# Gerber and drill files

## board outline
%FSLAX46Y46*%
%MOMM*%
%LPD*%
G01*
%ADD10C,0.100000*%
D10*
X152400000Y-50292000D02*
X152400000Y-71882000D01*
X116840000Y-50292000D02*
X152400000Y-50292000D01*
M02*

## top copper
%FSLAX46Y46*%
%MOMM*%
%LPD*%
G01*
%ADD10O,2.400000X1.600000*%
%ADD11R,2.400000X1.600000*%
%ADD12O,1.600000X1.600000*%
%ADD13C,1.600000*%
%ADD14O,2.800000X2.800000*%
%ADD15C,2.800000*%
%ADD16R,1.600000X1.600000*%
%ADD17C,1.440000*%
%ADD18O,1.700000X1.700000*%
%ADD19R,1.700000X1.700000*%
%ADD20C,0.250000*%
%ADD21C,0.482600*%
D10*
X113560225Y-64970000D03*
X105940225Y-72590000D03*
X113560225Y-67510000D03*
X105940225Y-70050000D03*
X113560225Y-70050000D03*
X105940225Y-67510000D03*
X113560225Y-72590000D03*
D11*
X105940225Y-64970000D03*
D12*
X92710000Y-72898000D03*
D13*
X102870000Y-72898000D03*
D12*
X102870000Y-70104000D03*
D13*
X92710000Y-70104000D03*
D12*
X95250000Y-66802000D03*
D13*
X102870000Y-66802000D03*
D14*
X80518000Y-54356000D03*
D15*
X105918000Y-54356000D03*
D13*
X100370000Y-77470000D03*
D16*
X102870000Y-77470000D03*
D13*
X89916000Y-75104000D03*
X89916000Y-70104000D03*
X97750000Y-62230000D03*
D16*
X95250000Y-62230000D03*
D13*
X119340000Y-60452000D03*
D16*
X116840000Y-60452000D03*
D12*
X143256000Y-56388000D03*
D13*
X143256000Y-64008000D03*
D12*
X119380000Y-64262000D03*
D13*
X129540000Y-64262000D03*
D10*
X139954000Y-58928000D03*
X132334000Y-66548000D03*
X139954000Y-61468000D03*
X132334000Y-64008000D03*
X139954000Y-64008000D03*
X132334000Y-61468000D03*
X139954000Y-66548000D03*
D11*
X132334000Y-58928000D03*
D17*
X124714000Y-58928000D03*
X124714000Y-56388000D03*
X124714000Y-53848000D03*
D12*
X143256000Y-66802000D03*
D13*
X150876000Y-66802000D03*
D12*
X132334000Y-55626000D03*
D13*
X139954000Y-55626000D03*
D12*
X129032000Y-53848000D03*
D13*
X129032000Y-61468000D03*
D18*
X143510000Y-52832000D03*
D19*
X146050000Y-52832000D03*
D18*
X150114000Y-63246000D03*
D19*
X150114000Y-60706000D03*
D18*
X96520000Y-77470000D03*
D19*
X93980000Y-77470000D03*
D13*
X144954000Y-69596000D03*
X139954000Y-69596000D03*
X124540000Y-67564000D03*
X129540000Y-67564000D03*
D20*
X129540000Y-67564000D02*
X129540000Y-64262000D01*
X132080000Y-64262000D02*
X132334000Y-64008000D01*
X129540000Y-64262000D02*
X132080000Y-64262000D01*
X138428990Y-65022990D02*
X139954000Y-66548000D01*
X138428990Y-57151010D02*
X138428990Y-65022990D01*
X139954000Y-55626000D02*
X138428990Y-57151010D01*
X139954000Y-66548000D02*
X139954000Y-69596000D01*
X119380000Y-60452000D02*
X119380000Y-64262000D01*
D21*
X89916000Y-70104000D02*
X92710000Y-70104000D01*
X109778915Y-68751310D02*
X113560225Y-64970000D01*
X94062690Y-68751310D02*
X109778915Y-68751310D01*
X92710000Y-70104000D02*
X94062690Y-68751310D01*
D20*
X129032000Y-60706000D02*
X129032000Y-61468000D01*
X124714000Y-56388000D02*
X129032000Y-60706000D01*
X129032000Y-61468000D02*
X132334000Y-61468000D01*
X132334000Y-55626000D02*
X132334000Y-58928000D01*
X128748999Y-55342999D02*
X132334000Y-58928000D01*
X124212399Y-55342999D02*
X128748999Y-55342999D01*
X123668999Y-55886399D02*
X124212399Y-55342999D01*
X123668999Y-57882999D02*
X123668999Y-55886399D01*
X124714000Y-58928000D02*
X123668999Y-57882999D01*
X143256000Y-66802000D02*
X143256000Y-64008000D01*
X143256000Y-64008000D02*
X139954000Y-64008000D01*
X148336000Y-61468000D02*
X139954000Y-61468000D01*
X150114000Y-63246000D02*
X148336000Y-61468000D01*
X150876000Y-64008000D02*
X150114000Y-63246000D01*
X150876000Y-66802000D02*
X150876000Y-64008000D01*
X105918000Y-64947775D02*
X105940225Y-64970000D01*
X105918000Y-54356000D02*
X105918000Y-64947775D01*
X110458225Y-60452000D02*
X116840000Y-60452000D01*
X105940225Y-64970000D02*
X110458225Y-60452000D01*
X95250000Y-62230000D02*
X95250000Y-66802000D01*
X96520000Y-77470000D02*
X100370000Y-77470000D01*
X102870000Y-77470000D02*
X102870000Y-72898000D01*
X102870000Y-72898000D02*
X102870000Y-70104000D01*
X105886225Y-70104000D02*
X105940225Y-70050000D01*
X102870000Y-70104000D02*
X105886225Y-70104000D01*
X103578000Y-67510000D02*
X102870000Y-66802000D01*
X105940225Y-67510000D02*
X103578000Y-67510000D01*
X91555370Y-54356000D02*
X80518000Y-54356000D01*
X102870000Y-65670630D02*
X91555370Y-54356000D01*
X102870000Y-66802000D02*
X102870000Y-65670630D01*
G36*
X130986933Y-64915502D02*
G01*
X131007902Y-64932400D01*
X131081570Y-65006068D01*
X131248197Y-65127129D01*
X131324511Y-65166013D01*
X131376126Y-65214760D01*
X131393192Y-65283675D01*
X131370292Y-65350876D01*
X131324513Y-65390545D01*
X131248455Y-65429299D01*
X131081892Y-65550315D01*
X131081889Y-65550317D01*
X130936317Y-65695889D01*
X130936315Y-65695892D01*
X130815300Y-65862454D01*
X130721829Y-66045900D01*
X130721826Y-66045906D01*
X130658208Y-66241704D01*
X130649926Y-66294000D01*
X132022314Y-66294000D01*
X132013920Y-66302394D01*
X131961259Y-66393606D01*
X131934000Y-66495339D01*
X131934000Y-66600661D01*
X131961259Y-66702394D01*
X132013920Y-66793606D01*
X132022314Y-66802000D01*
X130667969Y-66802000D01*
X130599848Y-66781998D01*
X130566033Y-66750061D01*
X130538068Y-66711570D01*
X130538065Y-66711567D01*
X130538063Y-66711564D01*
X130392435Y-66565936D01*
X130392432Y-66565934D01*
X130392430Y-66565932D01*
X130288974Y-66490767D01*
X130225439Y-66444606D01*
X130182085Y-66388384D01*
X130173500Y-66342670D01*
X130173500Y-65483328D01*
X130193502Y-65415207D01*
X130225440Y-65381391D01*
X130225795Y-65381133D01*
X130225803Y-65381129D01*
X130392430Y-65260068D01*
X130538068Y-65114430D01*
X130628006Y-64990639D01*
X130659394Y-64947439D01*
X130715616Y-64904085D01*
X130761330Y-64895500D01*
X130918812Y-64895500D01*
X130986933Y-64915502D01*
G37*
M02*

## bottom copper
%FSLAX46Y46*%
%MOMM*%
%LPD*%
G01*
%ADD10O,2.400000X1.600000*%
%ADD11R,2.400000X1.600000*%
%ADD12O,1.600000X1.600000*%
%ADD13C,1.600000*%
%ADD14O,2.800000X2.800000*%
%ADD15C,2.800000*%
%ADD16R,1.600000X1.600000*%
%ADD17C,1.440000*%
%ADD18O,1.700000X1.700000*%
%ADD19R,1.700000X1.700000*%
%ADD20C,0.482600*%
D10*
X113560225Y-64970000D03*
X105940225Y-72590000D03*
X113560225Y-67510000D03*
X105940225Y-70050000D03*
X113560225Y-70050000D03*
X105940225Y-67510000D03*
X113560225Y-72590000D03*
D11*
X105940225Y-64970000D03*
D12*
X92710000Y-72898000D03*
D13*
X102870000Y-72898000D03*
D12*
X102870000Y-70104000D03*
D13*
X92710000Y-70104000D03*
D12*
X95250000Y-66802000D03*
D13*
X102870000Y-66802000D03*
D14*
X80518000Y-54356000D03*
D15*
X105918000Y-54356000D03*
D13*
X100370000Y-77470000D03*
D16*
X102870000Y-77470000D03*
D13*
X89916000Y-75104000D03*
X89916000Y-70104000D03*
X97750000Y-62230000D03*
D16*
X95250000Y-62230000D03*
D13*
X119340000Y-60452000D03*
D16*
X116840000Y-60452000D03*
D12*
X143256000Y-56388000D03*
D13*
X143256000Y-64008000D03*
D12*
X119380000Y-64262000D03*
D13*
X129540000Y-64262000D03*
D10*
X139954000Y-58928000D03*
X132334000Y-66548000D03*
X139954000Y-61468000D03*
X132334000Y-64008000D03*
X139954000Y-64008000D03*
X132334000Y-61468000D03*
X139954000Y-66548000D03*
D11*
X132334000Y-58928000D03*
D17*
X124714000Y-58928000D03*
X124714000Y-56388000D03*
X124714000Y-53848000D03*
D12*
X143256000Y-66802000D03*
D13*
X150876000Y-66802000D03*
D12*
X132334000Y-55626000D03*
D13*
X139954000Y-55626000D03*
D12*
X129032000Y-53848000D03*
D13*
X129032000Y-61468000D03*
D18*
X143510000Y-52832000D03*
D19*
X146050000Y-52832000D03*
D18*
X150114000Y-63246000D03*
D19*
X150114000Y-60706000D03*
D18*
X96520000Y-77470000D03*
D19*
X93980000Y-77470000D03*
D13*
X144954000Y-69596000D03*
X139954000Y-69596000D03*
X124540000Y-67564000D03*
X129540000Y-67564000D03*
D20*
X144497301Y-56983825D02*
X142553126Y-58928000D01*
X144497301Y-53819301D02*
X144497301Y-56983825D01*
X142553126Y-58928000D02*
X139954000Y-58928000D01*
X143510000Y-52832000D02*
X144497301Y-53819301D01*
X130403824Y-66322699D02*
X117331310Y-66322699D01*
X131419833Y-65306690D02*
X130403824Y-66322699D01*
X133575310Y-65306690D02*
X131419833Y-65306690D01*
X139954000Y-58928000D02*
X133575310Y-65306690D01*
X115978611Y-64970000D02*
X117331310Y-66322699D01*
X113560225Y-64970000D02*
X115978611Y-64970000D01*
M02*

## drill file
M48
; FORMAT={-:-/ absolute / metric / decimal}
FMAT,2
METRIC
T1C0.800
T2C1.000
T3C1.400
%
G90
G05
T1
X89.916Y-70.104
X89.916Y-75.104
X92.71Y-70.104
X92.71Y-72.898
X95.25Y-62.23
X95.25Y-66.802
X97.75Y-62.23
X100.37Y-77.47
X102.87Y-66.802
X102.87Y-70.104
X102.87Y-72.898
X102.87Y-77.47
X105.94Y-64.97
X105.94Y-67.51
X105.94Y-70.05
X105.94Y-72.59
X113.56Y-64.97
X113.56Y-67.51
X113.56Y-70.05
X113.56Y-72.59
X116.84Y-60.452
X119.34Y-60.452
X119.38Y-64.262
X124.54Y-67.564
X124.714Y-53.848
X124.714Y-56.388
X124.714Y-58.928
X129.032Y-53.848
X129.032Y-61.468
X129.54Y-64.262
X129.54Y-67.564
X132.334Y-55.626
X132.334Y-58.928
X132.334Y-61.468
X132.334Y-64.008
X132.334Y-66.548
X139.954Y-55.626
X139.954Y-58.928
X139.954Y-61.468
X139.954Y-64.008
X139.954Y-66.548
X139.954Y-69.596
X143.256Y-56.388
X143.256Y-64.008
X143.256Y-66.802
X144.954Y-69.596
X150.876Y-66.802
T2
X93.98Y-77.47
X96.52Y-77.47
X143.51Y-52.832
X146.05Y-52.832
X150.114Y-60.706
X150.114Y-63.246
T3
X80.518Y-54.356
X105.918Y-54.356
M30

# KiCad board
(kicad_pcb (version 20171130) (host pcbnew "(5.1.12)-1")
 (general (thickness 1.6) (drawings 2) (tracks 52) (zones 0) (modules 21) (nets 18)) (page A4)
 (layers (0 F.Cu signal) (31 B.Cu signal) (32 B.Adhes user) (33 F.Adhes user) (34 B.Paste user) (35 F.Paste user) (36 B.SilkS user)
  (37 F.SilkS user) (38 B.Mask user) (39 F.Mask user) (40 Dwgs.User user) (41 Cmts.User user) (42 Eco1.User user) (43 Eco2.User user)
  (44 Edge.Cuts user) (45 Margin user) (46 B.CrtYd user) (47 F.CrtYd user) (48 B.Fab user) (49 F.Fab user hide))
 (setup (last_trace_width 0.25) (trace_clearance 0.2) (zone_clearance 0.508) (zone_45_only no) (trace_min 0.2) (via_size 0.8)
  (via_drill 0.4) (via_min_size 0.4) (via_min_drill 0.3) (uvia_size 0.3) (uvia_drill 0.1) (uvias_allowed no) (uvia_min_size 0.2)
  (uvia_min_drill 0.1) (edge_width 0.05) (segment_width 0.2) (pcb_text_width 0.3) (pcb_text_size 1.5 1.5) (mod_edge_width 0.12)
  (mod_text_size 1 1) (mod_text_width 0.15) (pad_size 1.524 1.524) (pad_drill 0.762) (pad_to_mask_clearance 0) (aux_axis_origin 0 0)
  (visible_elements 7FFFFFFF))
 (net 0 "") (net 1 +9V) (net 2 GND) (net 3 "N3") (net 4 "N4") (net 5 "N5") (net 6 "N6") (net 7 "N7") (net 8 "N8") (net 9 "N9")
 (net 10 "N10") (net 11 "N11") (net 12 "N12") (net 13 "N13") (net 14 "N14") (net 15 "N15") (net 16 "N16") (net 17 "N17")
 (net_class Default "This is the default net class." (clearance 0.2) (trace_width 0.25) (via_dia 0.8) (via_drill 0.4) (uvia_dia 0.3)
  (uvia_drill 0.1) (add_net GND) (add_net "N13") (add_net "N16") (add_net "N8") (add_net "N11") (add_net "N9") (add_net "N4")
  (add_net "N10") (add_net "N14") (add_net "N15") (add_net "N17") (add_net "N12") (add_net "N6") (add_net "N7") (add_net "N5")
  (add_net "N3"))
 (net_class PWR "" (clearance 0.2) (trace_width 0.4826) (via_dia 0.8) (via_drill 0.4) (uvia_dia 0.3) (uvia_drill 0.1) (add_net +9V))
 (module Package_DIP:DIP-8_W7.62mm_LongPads (layer F.Cu) (at 105.940225 64.97)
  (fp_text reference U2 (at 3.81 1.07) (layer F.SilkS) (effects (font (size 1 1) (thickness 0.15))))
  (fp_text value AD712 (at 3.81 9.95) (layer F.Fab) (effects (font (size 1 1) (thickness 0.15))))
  (pad 8 thru_hole oval (at 7.62 0) (size 2.4 1.6) (drill 0.8) (layers *.Cu *.Mask) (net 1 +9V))
  (pad 4 thru_hole oval (at 0 7.62) (size 2.4 1.6) (drill 0.8) (layers *.Cu *.Mask) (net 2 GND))
  (pad 7 thru_hole oval (at 7.62 2.54) (size 2.4 1.6) (drill 0.8) (layers *.Cu *.Mask) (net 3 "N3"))
  (pad 3 thru_hole oval (at 0 5.08) (size 2.4 1.6) (drill 0.8) (layers *.Cu *.Mask) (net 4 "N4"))
  (pad 6 thru_hole oval (at 7.62 5.08) (size 2.4 1.6) (drill 0.8) (layers *.Cu *.Mask) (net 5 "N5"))
  (pad 2 thru_hole oval (at 0 2.54) (size 2.4 1.6) (drill 0.8) (layers *.Cu *.Mask) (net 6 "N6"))
  (pad 5 thru_hole oval (at 7.62 7.62) (size 2.4 1.6) (drill 0.8) (layers *.Cu *.Mask) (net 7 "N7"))
  (pad 1 thru_hole rect (at 0 0) (size 2.4 1.6) (drill 0.8) (layers *.Cu *.Mask) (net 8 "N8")))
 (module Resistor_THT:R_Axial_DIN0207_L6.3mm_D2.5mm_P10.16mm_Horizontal (layer F.Cu) (at 102.87 72.898 180)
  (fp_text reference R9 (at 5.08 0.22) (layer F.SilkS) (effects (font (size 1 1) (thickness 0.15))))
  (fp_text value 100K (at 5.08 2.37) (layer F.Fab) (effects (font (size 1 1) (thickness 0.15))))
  (pad 2 thru_hole oval (at 10.16 0 180) (size 1.6 1.6) (drill 0.8) (layers *.Cu *.Mask) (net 2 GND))
  (pad 1 thru_hole circle (at 0 0 180) (size 1.6 1.6) (drill 0.8) (layers *.Cu *.Mask) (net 4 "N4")))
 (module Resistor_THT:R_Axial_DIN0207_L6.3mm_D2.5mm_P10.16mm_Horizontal (layer F.Cu) (at 92.71 70.104)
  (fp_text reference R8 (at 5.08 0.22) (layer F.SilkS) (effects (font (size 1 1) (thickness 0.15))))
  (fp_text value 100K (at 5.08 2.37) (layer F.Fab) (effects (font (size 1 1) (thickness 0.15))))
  (pad 2 thru_hole oval (at 10.16 0) (size 1.6 1.6) (drill 0.8) (layers *.Cu *.Mask) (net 4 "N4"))
  (pad 1 thru_hole circle (at 0 0) (size 1.6 1.6) (drill 0.8) (layers *.Cu *.Mask) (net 1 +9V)))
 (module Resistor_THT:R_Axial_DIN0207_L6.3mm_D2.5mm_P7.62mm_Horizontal (layer F.Cu) (at 102.87 66.802 180)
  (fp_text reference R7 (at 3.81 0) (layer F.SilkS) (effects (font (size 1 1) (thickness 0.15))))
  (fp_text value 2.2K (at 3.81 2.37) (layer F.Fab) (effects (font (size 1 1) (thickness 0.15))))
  (pad 2 thru_hole oval (at 7.62 0 180) (size 1.6 1.6) (drill 0.8) (layers *.Cu *.Mask) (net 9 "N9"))
  (pad 1 thru_hole circle (at 0 0 180) (size 1.6 1.6) (drill 0.8) (layers *.Cu *.Mask) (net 6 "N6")))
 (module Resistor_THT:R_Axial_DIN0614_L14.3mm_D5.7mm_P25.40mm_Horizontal (layer F.Cu) (at 105.918 54.356 180)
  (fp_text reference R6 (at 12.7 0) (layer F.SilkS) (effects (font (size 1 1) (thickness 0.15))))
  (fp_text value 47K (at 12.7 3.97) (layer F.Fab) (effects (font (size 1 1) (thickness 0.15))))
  (pad 2 thru_hole oval (at 25.4 0 180) (size 2.8 2.8) (drill 1.4) (layers *.Cu *.Mask) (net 6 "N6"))
  (pad 1 thru_hole circle (at 0 0 180) (size 2.8 2.8) (drill 1.4) (layers *.Cu *.Mask) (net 8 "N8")))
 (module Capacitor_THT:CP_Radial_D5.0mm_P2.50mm (layer F.Cu) (at 102.87 77.47 180)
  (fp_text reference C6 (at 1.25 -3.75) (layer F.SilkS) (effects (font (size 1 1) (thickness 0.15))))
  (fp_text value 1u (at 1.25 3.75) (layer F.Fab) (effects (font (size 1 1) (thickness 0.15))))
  (pad 2 thru_hole circle (at 2.5 0 180) (size 1.6 1.6) (drill 0.8) (layers *.Cu *.Mask) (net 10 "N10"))
  (pad 1 thru_hole rect (at 0 0 180) (size 1.6 1.6) (drill 0.8) (layers *.Cu *.Mask) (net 4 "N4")))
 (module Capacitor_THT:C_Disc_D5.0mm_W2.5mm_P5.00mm (layer F.Cu) (at 89.916 70.104 270)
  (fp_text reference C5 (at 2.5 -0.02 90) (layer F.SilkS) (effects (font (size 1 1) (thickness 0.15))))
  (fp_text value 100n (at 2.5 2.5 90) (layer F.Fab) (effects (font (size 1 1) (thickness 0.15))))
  (pad 2 thru_hole circle (at 5 0 270) (size 1.6 1.6) (drill 0.8) (layers *.Cu *.Mask) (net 2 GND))
  (pad 1 thru_hole circle (at 0 0 270) (size 1.6 1.6) (drill 0.8) (layers *.Cu *.Mask) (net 1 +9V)))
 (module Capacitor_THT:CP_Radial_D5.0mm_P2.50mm (layer F.Cu) (at 95.25 62.23)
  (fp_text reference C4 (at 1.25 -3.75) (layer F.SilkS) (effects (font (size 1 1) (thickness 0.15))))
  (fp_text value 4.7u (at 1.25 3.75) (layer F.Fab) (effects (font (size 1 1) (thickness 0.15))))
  (pad 2 thru_hole circle (at 2.5 0) (size 1.6 1.6) (drill 0.8) (layers *.Cu *.Mask) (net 2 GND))
  (pad 1 thru_hole rect (at 0 0) (size 1.6 1.6) (drill 0.8) (layers *.Cu *.Mask) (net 9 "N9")))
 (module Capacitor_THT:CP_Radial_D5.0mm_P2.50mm (layer F.Cu) (at 116.84 60.452)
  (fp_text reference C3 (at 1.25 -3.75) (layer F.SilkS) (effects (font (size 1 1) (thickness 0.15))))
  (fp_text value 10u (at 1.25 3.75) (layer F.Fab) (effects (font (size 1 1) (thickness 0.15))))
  (pad 2 thru_hole circle (at 2.5 0) (size 1.6 1.6) (drill 0.8) (layers *.Cu *.Mask) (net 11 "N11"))
  (pad 1 thru_hole rect (at 0 0) (size 1.6 1.6) (drill 0.8) (layers *.Cu *.Mask) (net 8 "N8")))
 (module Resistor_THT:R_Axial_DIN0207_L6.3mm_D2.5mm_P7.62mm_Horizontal (layer F.Cu) (at 143.256 64.008 90)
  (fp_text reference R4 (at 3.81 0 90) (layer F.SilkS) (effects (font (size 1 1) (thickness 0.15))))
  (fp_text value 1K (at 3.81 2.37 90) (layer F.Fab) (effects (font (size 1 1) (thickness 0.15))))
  (pad 2 thru_hole oval (at 7.62 0 90) (size 1.6 1.6) (drill 0.8) (layers *.Cu *.Mask) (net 2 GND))
  (pad 1 thru_hole circle (at 0 0 90) (size 1.6 1.6) (drill 0.8) (layers *.Cu *.Mask) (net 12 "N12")))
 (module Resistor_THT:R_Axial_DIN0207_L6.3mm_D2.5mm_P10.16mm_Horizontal (layer F.Cu) (at 129.54 64.262 180)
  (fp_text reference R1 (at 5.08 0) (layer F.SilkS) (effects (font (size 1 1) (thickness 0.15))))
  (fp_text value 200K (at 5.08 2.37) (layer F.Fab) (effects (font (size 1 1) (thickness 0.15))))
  (pad 2 thru_hole oval (at 10.16 0 180) (size 1.6 1.6) (drill 0.8) (layers *.Cu *.Mask) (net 11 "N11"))
  (pad 1 thru_hole circle (at 0 0 180) (size 1.6 1.6) (drill 0.8) (layers *.Cu *.Mask) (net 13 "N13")))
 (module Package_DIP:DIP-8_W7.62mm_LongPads (layer F.Cu) (at 132.334 58.928)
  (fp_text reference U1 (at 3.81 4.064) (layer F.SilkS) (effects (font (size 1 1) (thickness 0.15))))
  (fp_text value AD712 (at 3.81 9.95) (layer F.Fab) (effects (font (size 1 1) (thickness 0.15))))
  (pad 8 thru_hole oval (at 7.62 0) (size 2.4 1.6) (drill 0.8) (layers *.Cu *.Mask) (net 1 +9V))
  (pad 4 thru_hole oval (at 0 7.62) (size 2.4 1.6) (drill 0.8) (layers *.Cu *.Mask) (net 2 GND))
  (pad 7 thru_hole oval (at 7.62 2.54) (size 2.4 1.6) (drill 0.8) (layers *.Cu *.Mask) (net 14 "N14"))
  (pad 3 thru_hole oval (at 0 5.08) (size 2.4 1.6) (drill 0.8) (layers *.Cu *.Mask) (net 13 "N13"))
  (pad 6 thru_hole oval (at 7.62 5.08) (size 2.4 1.6) (drill 0.8) (layers *.Cu *.Mask) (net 12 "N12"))
  (pad 2 thru_hole oval (at 0 2.54) (size 2.4 1.6) (drill 0.8) (layers *.Cu *.Mask) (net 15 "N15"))
  (pad 5 thru_hole oval (at 7.62 7.62) (size 2.4 1.6) (drill 0.8) (layers *.Cu *.Mask) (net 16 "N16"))
  (pad 1 thru_hole rect (at 0 0) (size 2.4 1.6) (drill 0.8) (layers *.Cu *.Mask) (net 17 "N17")))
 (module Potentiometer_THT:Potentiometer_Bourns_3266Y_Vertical (layer F.Cu) (at 124.714 53.848 90)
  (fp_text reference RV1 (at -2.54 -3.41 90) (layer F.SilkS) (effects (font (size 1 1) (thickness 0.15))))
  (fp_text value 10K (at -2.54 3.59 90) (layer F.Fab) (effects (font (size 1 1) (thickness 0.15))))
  (pad 3 thru_hole circle (at -5.08 0 90) (size 1.44 1.44) (drill 0.8) (layers *.Cu *.Mask) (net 17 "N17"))
  (pad 2 thru_hole circle (at -2.54 0 90) (size 1.44 1.44) (drill 0.8) (layers *.Cu *.Mask) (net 15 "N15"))
  (pad 1 thru_hole circle (at 0 0 90) (size 1.44 1.44) (drill 0.8) (layers *.Cu *.Mask) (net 2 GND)))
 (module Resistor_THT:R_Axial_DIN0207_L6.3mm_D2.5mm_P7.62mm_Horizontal (layer F.Cu) (at 150.876 66.802 180)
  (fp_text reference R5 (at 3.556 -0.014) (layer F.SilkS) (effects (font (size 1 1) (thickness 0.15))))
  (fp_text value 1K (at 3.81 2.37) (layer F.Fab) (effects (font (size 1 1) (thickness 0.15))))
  (pad 2 thru_hole oval (at 7.62 0 180) (size 1.6 1.6) (drill 0.8) (layers *.Cu *.Mask) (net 12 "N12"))
  (pad 1 thru_hole circle (at 0 0 180) (size 1.6 1.6) (drill 0.8) (layers *.Cu *.Mask) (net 14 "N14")))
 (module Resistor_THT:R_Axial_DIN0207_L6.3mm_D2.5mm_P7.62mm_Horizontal (layer F.Cu) (at 139.954 55.626 180)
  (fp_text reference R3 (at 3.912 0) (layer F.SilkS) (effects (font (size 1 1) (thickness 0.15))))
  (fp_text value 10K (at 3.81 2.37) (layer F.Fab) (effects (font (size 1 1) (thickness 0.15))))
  (pad 2 thru_hole oval (at 7.62 0 180) (size 1.6 1.6) (drill 0.8) (layers *.Cu *.Mask) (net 17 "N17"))
  (pad 1 thru_hole circle (at 0 0 180) (size 1.6 1.6) (drill 0.8) (layers *.Cu *.Mask) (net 16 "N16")))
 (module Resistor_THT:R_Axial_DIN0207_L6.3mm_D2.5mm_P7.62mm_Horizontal (layer F.Cu) (at 129.032 61.468 90)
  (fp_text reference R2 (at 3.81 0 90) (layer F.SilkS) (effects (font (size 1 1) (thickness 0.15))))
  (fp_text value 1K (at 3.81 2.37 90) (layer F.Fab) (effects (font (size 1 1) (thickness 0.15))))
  (pad 2 thru_hole oval (at 7.62 0 90) (size 1.6 1.6) (drill 0.8) (layers *.Cu *.Mask) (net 2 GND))
  (pad 1 thru_hole circle (at 0 0 90) (size 1.6 1.6) (drill 0.8) (layers *.Cu *.Mask) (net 15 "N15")))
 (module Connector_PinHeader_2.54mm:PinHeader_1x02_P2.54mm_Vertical (layer F.Cu) (at 146.05 52.832 270)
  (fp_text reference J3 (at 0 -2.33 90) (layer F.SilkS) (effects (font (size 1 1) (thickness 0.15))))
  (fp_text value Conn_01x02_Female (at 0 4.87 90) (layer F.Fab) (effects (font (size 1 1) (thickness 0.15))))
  (pad 2 thru_hole oval (at 0 2.54 270) (size 1.7 1.7) (drill 1) (layers *.Cu *.Mask) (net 1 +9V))
  (pad 1 thru_hole rect (at 0 0 270) (size 1.7 1.7) (drill 1) (layers *.Cu *.Mask) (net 2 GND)))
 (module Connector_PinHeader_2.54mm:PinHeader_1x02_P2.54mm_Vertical (layer F.Cu) (at 150.114 60.706)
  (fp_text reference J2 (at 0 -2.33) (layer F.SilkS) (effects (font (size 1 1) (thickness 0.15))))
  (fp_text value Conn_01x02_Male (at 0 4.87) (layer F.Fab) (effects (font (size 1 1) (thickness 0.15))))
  (pad 2 thru_hole oval (at 0 2.54) (size 1.7 1.7) (drill 1) (layers *.Cu *.Mask) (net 14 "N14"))
  (pad 1 thru_hole rect (at 0 0) (size 1.7 1.7) (drill 1) (layers *.Cu *.Mask) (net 2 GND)))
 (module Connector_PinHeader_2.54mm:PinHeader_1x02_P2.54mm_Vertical (layer F.Cu) (at 93.98 77.47 90)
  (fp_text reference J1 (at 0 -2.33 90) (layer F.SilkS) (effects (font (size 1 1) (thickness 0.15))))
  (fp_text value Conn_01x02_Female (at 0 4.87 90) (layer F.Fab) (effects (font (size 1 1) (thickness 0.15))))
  (pad 2 thru_hole oval (at 0 2.54 90) (size 1.7 1.7) (drill 1) (layers *.Cu *.Mask) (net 10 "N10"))
  (pad 1 thru_hole rect (at 0 0 90) (size 1.7 1.7) (drill 1) (layers *.Cu *.Mask) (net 2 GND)))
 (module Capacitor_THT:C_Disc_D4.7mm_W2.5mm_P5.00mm (layer F.Cu) (at 139.954 69.596)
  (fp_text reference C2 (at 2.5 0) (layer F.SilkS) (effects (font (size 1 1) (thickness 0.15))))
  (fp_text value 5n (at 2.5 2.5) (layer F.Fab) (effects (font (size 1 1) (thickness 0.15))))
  (pad 2 thru_hole circle (at 5 0) (size 1.6 1.6) (drill 0.8) (layers *.Cu *.Mask) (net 2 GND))
  (pad 1 thru_hole circle (at 0 0) (size 1.6 1.6) (drill 0.8) (layers *.Cu *.Mask) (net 16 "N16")))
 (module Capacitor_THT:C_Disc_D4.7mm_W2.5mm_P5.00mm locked (layer F.Cu) (at 129.54 67.564 180)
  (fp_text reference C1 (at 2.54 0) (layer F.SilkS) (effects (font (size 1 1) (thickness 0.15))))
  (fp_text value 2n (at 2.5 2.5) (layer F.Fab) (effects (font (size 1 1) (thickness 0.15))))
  (pad 2 thru_hole circle (at 5 0 180) (size 1.6 1.6) (drill 0.8) (layers *.Cu *.Mask) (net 2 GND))
  (pad 1 thru_hole circle (at 0 0 180) (size 1.6 1.6) (drill 0.8) (layers *.Cu *.Mask) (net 13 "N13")))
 (gr_line (start 152.4 50.292) (end 152.4 71.882) (layer Edge.Cuts) (width 0.1))
 (gr_line (start 116.84 50.292) (end 152.4 50.292) (layer Edge.Cuts) (width 0.1))
 (segment (start 129.54 67.564) (end 129.54 64.262) (width 0.25) (layer F.Cu) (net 13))
 (segment (start 132.08 64.262) (end 132.334 64.008) (width 0.25) (layer F.Cu) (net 13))
 (segment (start 129.54 64.262) (end 132.08 64.262) (width 0.25) (layer F.Cu) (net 13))
 (segment (start 138.42899 65.02299) (end 139.954 66.548) (width 0.25) (layer F.Cu) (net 16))
 (segment (start 138.42899 57.15101) (end 138.42899 65.02299) (width 0.25) (layer F.Cu) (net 16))
 (segment (start 139.954 55.626) (end 138.42899 57.15101) (width 0.25) (layer F.Cu) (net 16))
 (segment (start 139.954 66.548) (end 139.954 69.596) (width 0.25) (layer F.Cu) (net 16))
 (segment (start 119.38 60.452) (end 119.38 64.262) (width 0.25) (layer F.Cu) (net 11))
 (segment (start 144.497301 56.983825) (end 142.553126 58.928) (width 0.4826) (layer B.Cu) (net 1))
 (segment (start 144.497301 53.819301) (end 144.497301 56.983825) (width 0.4826) (layer B.Cu) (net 1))
 (segment (start 142.553126 58.928) (end 139.954 58.928) (width 0.4826) (layer B.Cu) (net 1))
 (segment (start 143.51 52.832) (end 144.497301 53.819301) (width 0.4826) (layer B.Cu) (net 1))
 (segment (start 89.916 70.104) (end 92.71 70.104) (width 0.4826) (layer F.Cu) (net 1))
 (segment (start 109.778915 68.75131) (end 113.560225 64.97) (width 0.4826) (layer F.Cu) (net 1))
 (segment (start 94.06269 68.75131) (end 109.778915 68.75131) (width 0.4826) (layer F.Cu) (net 1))
 (segment (start 92.71 70.104) (end 94.06269 68.75131) (width 0.4826) (layer F.Cu) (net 1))
 (segment (start 130.403824 66.322699) (end 117.33131 66.322699) (width 0.4826) (layer B.Cu) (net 1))
 (segment (start 131.419833 65.30669) (end 130.403824 66.322699) (width 0.4826) (layer B.Cu) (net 1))
 (segment (start 133.57531 65.30669) (end 131.419833 65.30669) (width 0.4826) (layer B.Cu) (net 1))
 (segment (start 139.954 58.928) (end 133.57531 65.30669) (width 0.4826) (layer B.Cu) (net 1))
 (segment (start 115.978611 64.97) (end 117.33131 66.322699) (width 0.4826) (layer B.Cu) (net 1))
 (segment (start 113.560225 64.97) (end 115.978611 64.97) (width 0.4826) (layer B.Cu) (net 1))
 (segment (start 129.032 60.706) (end 129.032 61.468) (width 0.25) (layer F.Cu) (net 15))
 (segment (start 124.714 56.388) (end 129.032 60.706) (width 0.25) (layer F.Cu) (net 15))
 (segment (start 129.032 61.468) (end 132.334 61.468) (width 0.25) (layer F.Cu) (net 15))
 (segment (start 132.334 55.626) (end 132.334 58.928) (width 0.25) (layer F.Cu) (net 17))
 (segment (start 128.748999 55.342999) (end 132.334 58.928) (width 0.25) (layer F.Cu) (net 17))
 (segment (start 124.212399 55.342999) (end 128.748999 55.342999) (width 0.25) (layer F.Cu) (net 17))
 (segment (start 123.668999 55.886399) (end 124.212399 55.342999) (width 0.25) (layer F.Cu) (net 17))
 (segment (start 123.668999 57.882999) (end 123.668999 55.886399) (width 0.25) (layer F.Cu) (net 17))
 (segment (start 124.714 58.928) (end 123.668999 57.882999) (width 0.25) (layer F.Cu) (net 17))
 (segment (start 143.256 66.802) (end 143.256 64.008) (width 0.25) (layer F.Cu) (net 12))
 (segment (start 143.256 64.008) (end 139.954 64.008) (width 0.25) (layer F.Cu) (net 12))
 (segment (start 148.336 61.468) (end 139.954 61.468) (width 0.25) (layer F.Cu) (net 14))
 (segment (start 150.114 63.246) (end 148.336 61.468) (width 0.25) (layer F.Cu) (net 14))
 (segment (start 150.876 64.008) (end 150.114 63.246) (width 0.25) (layer F.Cu) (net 14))
 (segment (start 150.876 66.802) (end 150.876 64.008) (width 0.25) (layer F.Cu) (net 14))
 (segment (start 105.918 64.947775) (end 105.940225 64.97) (width 0.25) (layer F.Cu) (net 8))
 (segment (start 105.918 54.356) (end 105.918 64.947775) (width 0.25) (layer F.Cu) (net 8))
 (segment (start 110.458225 60.452) (end 116.84 60.452) (width 0.25) (layer F.Cu) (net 8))
 (segment (start 105.940225 64.97) (end 110.458225 60.452) (width 0.25) (layer F.Cu) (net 8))
 (segment (start 95.25 62.23) (end 95.25 66.802) (width 0.25) (layer F.Cu) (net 9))
 (segment (start 96.52 77.47) (end 100.37 77.47) (width 0.25) (layer F.Cu) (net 10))
 (segment (start 102.87 77.47) (end 102.87 72.898) (width 0.25) (layer F.Cu) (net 4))
 (segment (start 102.87 72.898) (end 102.87 70.104) (width 0.25) (layer F.Cu) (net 4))
 (segment (start 105.886225 70.104) (end 105.940225 70.05) (width 0.25) (layer F.Cu) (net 4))
 (segment (start 102.87 70.104) (end 105.886225 70.104) (width 0.25) (layer F.Cu) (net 4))
 (segment (start 103.578 67.51) (end 102.87 66.802) (width 0.25) (layer F.Cu) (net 6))
 (segment (start 105.940225 67.51) (end 103.578 67.51) (width 0.25) (layer F.Cu) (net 6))
 (segment (start 91.55537 54.356) (end 80.518 54.356) (width 0.25) (layer F.Cu) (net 6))
 (segment (start 102.87 65.67063) (end 91.55537 54.356) (width 0.25) (layer F.Cu) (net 6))
 (segment (start 102.87 66.802) (end 102.87 65.67063) (width 0.25) (layer F.Cu) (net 6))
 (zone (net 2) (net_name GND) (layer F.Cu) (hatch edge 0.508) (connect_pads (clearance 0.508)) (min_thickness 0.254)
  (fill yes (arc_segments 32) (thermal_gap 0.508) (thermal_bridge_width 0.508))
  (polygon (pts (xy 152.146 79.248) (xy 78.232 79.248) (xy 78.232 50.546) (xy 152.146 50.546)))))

